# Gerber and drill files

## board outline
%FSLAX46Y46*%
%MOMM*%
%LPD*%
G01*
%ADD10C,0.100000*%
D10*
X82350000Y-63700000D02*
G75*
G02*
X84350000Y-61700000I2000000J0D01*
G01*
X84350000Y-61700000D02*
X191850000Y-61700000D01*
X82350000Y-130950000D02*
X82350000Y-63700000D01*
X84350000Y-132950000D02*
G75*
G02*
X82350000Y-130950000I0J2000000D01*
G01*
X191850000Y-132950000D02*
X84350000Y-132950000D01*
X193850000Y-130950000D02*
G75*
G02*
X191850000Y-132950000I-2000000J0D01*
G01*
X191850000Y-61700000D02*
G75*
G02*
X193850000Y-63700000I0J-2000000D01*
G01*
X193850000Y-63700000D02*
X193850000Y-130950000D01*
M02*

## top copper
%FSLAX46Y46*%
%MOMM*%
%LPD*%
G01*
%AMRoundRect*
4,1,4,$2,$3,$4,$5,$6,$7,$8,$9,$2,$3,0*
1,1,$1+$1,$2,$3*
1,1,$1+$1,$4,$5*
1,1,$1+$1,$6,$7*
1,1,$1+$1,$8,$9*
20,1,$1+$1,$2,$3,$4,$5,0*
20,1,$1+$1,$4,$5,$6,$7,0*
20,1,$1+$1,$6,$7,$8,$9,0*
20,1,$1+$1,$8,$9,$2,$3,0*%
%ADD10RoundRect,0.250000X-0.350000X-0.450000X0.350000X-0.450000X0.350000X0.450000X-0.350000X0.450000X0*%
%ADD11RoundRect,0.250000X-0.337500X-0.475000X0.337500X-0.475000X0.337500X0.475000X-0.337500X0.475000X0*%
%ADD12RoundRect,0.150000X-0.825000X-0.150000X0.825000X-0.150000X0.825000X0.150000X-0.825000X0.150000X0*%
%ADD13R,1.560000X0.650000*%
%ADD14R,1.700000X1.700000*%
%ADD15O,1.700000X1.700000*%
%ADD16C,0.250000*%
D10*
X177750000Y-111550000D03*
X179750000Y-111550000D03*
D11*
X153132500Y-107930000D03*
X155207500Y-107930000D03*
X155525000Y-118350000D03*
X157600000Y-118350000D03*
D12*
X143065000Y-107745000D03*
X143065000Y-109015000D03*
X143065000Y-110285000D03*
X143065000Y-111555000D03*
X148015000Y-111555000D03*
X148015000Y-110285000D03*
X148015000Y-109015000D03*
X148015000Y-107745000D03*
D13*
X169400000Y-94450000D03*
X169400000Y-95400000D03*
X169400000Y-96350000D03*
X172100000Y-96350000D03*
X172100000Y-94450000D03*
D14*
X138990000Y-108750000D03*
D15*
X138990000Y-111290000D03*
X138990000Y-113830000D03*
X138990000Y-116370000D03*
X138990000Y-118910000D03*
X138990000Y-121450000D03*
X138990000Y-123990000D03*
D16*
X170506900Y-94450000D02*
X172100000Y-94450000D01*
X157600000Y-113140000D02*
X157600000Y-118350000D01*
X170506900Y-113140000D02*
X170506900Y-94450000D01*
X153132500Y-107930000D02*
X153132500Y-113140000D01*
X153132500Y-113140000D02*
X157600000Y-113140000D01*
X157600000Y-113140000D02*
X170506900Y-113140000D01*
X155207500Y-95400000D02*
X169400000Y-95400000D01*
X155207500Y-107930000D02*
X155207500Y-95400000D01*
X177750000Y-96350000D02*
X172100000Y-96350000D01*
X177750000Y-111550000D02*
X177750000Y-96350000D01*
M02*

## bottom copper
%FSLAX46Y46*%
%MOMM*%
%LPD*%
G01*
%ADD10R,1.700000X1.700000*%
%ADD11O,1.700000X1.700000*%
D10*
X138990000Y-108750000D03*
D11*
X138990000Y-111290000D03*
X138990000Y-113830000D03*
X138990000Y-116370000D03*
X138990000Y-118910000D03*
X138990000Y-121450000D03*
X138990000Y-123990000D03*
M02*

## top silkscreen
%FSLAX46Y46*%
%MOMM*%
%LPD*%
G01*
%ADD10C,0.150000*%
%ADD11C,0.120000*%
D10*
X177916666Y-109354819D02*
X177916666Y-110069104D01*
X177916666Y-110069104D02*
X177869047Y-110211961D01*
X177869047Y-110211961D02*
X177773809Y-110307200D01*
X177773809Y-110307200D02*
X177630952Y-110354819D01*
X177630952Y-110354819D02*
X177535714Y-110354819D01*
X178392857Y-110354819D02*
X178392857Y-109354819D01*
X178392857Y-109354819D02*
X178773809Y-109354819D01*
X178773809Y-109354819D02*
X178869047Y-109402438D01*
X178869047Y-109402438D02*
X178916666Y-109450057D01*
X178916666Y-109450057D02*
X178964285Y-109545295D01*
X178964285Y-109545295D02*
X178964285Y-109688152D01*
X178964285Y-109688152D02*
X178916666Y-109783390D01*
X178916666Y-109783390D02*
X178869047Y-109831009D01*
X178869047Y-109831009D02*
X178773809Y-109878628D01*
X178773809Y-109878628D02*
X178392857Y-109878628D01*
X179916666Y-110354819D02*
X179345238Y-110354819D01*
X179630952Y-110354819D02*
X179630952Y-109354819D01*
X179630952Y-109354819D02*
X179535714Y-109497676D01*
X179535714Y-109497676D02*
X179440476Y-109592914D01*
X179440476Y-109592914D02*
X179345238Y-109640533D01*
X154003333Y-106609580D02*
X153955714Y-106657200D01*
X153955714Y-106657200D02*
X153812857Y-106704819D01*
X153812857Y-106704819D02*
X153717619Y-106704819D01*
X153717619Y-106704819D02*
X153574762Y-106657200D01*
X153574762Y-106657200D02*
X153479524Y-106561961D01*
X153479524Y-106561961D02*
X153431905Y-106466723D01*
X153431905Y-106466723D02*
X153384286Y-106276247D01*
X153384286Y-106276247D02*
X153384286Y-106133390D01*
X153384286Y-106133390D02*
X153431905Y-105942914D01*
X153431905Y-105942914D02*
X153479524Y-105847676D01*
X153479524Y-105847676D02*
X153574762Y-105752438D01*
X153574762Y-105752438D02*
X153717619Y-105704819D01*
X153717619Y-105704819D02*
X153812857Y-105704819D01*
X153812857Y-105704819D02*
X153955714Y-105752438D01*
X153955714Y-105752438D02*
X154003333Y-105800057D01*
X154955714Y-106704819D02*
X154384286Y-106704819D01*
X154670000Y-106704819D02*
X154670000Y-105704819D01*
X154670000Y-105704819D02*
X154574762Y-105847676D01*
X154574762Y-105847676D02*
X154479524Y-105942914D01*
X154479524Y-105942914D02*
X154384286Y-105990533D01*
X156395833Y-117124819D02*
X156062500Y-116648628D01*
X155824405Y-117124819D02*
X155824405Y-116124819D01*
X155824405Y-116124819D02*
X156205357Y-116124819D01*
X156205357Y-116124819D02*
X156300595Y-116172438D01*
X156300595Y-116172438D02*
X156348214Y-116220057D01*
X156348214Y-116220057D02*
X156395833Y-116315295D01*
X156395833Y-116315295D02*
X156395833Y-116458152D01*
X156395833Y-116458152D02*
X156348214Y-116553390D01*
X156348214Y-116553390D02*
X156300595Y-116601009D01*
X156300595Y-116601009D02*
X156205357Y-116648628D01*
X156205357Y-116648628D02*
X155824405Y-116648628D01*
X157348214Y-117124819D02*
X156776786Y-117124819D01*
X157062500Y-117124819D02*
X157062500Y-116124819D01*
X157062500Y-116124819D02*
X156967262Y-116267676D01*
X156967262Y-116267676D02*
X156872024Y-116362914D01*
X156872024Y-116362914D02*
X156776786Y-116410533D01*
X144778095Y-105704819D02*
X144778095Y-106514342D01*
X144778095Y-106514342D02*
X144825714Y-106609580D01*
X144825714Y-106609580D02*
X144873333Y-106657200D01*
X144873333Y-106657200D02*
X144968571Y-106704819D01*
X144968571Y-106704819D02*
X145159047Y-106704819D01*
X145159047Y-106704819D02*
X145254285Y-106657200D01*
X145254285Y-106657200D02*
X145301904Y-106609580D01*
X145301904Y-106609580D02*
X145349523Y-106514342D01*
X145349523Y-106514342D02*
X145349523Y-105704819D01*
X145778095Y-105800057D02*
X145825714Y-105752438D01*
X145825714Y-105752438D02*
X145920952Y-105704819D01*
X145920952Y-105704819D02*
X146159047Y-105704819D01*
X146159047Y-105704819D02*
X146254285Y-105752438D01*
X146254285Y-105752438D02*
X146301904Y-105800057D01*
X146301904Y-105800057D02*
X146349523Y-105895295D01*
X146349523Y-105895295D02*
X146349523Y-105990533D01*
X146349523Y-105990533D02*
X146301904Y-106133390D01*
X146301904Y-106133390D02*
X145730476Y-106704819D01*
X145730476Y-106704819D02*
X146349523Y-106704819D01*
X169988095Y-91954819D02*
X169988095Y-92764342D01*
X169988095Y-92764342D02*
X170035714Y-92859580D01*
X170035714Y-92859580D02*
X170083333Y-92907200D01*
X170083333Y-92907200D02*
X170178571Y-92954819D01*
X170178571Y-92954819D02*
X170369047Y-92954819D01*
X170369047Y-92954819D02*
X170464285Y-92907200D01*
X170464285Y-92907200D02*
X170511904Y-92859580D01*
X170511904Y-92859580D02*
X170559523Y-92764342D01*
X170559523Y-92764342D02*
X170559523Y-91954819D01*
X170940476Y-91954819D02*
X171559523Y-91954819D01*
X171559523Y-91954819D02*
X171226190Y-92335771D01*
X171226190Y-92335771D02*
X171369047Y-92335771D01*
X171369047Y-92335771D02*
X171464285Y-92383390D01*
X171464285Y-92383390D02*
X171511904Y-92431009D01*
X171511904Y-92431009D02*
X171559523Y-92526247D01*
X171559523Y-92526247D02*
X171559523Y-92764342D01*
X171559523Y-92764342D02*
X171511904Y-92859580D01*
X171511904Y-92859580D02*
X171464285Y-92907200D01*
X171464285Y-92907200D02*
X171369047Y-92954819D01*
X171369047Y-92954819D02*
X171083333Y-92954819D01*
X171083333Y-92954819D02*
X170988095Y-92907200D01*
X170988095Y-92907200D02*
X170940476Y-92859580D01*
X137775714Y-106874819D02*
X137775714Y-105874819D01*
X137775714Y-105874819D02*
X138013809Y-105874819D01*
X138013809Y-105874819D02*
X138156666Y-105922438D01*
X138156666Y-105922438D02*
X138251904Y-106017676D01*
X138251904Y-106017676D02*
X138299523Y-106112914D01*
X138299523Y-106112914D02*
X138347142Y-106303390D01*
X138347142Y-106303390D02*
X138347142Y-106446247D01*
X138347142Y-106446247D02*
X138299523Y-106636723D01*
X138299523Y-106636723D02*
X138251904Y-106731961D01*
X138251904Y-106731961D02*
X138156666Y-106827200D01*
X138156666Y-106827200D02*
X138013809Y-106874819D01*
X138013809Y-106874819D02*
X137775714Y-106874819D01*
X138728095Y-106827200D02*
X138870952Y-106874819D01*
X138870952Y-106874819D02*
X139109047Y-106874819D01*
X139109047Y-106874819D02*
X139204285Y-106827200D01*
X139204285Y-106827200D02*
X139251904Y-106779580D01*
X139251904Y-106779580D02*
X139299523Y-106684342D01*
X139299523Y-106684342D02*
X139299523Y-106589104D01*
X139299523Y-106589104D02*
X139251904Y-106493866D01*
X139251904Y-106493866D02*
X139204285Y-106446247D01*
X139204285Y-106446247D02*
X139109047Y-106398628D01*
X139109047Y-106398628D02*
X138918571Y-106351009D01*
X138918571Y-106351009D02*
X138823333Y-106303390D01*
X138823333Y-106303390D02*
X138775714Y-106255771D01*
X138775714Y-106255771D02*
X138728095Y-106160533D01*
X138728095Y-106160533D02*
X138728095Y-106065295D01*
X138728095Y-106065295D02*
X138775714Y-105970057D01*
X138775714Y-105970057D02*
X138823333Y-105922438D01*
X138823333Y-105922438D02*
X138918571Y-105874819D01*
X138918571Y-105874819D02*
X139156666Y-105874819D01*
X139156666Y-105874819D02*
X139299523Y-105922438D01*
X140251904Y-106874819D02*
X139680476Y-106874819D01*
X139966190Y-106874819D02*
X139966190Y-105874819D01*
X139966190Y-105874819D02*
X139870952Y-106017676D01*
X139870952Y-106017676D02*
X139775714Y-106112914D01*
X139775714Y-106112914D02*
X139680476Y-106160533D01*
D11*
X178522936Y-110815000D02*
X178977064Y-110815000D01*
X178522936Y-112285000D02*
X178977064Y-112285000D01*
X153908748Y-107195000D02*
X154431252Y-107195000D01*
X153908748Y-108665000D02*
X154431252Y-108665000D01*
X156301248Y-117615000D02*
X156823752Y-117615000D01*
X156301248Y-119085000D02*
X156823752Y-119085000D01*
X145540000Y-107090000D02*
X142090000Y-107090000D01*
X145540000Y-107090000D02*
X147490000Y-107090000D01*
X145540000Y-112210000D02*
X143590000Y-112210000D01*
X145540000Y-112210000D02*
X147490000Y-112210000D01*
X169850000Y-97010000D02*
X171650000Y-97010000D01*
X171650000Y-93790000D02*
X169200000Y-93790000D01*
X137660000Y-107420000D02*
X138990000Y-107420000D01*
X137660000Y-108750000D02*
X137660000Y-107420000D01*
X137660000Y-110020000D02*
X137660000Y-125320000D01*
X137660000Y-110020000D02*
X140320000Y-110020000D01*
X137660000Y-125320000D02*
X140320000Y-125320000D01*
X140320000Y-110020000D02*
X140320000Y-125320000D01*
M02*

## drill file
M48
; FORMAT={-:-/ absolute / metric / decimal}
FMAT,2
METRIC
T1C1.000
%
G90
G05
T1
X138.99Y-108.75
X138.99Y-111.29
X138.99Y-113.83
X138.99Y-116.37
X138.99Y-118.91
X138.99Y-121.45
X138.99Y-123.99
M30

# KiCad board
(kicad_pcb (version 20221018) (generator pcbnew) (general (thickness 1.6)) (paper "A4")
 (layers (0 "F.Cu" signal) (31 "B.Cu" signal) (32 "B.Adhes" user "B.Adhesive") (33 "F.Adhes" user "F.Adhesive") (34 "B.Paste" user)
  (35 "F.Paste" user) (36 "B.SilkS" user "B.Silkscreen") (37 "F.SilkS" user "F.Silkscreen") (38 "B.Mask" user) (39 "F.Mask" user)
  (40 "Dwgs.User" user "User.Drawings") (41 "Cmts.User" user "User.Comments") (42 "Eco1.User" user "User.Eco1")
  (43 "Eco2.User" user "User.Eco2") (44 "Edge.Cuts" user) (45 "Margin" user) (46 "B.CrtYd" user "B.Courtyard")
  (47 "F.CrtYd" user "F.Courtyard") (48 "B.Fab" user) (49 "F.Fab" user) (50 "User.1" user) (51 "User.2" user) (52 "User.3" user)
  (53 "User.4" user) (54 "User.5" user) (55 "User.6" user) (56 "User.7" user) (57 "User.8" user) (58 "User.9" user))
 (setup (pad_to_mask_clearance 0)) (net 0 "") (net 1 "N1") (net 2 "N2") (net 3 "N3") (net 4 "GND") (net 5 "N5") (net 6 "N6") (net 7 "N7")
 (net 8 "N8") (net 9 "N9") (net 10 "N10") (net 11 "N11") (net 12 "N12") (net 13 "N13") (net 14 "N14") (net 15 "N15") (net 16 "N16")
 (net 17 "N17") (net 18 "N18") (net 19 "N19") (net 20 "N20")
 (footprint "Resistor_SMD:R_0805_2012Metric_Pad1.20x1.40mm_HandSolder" (layer "F.Cu") (at 178.75 111.55)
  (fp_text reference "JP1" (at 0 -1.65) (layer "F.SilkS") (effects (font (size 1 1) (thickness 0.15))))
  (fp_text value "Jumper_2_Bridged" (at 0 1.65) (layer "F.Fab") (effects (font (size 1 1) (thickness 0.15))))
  (fp_line (start -0.227064 -0.735) (end 0.227064 -0.735) (stroke (width 0.12) (type solid)) (layer "F.SilkS"))
  (fp_line (start -0.227064 0.735) (end 0.227064 0.735) (stroke (width 0.12) (type solid)) (layer "F.SilkS"))
  (pad "1" smd roundrect (at -1 0) (size 1.2 1.4) (layers "F.Cu" "F.Paste" "F.Mask") (roundrect_rratio 0.208333) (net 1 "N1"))
  (pad "2" smd roundrect (at 1 0) (size 1.2 1.4) (layers "F.Cu" "F.Paste" "F.Mask") (roundrect_rratio 0.208333) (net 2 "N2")))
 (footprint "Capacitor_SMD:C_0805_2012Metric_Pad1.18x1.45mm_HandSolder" (layer "F.Cu") (at 154.17 107.93)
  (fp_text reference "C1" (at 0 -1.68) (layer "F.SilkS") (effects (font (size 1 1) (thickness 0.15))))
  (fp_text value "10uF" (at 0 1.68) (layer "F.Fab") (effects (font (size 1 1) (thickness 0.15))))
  (fp_line (start -0.261252 -0.735) (end 0.261252 -0.735) (stroke (width 0.12) (type solid)) (layer "F.SilkS"))
  (fp_line (start -0.261252 0.735) (end 0.261252 0.735) (stroke (width 0.12) (type solid)) (layer "F.SilkS"))
  (pad "1" smd roundrect (at -1.0375 0) (size 1.175 1.45) (layers "F.Cu" "F.Paste" "F.Mask") (roundrect_rratio 0.212766) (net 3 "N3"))
  (pad "2" smd roundrect (at 1.0375 0) (size 1.175 1.45) (layers "F.Cu" "F.Paste" "F.Mask") (roundrect_rratio 0.212766) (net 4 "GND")))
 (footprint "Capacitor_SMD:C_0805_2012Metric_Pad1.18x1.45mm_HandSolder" (layer "F.Cu") (at 156.5625 118.35)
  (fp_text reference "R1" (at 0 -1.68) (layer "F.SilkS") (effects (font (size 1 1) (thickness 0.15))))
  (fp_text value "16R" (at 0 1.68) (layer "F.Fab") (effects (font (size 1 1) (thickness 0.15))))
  (fp_line (start -0.261252 -0.735) (end 0.261252 -0.735) (stroke (width 0.12) (type solid)) (layer "F.SilkS"))
  (fp_line (start -0.261252 0.735) (end 0.261252 0.735) (stroke (width 0.12) (type solid)) (layer "F.SilkS"))
  (pad "1" smd roundrect (at -1.0375 0) (size 1.175 1.45) (layers "F.Cu" "F.Paste" "F.Mask") (roundrect_rratio 0.212766) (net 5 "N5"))
  (pad "2" smd roundrect (at 1.0375 0) (size 1.175 1.45) (layers "F.Cu" "F.Paste" "F.Mask") (roundrect_rratio 0.212766) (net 3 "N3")))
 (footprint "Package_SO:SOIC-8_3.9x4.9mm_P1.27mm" (layer "F.Cu") (at 145.54 109.65)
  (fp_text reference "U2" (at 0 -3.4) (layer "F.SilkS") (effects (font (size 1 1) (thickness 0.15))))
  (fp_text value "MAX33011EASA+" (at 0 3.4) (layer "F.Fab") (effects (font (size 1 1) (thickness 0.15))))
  (fp_line (start 0 -2.56) (end -3.45 -2.56) (stroke (width 0.12) (type solid)) (layer "F.SilkS"))
  (fp_line (start 0 -2.56) (end 1.95 -2.56) (stroke (width 0.12) (type solid)) (layer "F.SilkS"))
  (fp_line (start 0 2.56) (end -1.95 2.56) (stroke (width 0.12) (type solid)) (layer "F.SilkS"))
  (fp_line (start 0 2.56) (end 1.95 2.56) (stroke (width 0.12) (type solid)) (layer "F.SilkS"))
  (pad "1" smd roundrect (at -2.475 -1.905) (size 1.95 0.6) (layers "F.Cu" "F.Paste" "F.Mask") (roundrect_rratio 0.25) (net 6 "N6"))
  (pad "2" smd roundrect (at -2.475 -0.635) (size 1.95 0.6) (layers "F.Cu" "F.Paste" "F.Mask") (roundrect_rratio 0.25) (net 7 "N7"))
  (pad "3" smd roundrect (at -2.475 0.635) (size 1.95 0.6) (layers "F.Cu" "F.Paste" "F.Mask") (roundrect_rratio 0.25) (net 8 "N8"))
  (pad "4" smd roundrect (at -2.475 1.905) (size 1.95 0.6) (layers "F.Cu" "F.Paste" "F.Mask") (roundrect_rratio 0.25) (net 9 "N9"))
  (pad "5" smd roundrect (at 2.475 1.905) (size 1.95 0.6) (layers "F.Cu" "F.Paste" "F.Mask") (roundrect_rratio 0.25) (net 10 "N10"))
  (pad "6" smd roundrect (at 2.475 0.635) (size 1.95 0.6) (layers "F.Cu" "F.Paste" "F.Mask") (roundrect_rratio 0.25) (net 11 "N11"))
  (pad "7" smd roundrect (at 2.475 -0.635) (size 1.95 0.6) (layers "F.Cu" "F.Paste" "F.Mask") (roundrect_rratio 0.25) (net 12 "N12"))
  (pad "8" smd roundrect (at 2.475 -1.905) (size 1.95 0.6) (layers "F.Cu" "F.Paste" "F.Mask") (roundrect_rratio 0.25) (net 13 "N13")))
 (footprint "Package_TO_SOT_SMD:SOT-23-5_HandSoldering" (layer "F.Cu") (at 170.75 95.4)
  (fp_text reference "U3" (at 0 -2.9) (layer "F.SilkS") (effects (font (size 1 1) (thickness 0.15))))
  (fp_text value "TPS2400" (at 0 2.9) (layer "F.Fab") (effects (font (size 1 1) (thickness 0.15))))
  (fp_line (start -0.9 1.61) (end 0.9 1.61) (stroke (width 0.12) (type solid)) (layer "F.SilkS"))
  (fp_line (start 0.9 -1.61) (end -1.55 -1.61) (stroke (width 0.12) (type solid)) (layer "F.SilkS"))
  (pad "1" smd rect (at -1.35 -0.95) (size 1.56 0.65) (layers "F.Cu" "F.Paste" "F.Mask"))
  (pad "2" smd rect (at -1.35 0) (size 1.56 0.65) (layers "F.Cu" "F.Paste" "F.Mask") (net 4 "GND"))
  (pad "3" smd rect (at -1.35 0.95) (size 1.56 0.65) (layers "F.Cu" "F.Paste" "F.Mask"))
  (pad "4" smd rect (at 1.35 0.95) (size 1.56 0.65) (layers "F.Cu" "F.Paste" "F.Mask") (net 1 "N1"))
  (pad "5" smd rect (at 1.35 -0.95) (size 1.56 0.65) (layers "F.Cu" "F.Paste" "F.Mask") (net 3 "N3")))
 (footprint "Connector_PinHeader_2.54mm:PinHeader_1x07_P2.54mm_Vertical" (layer "F.Cu") (at 138.99 108.75)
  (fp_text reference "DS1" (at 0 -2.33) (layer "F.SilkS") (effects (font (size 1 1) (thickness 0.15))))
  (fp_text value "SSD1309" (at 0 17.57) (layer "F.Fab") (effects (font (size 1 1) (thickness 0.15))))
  (fp_line (start -1.33 -1.33) (end 0 -1.33) (stroke (width 0.12) (type solid)) (layer "F.SilkS"))
  (fp_line (start -1.33 0) (end -1.33 -1.33) (stroke (width 0.12) (type solid)) (layer "F.SilkS"))
  (fp_line (start -1.33 1.27) (end -1.33 16.57) (stroke (width 0.12) (type solid)) (layer "F.SilkS"))
  (fp_line (start -1.33 1.27) (end 1.33 1.27) (stroke (width 0.12) (type solid)) (layer "F.SilkS"))
  (fp_line (start -1.33 16.57) (end 1.33 16.57) (stroke (width 0.12) (type solid)) (layer "F.SilkS"))
  (fp_line (start 1.33 1.27) (end 1.33 16.57) (stroke (width 0.12) (type solid)) (layer "F.SilkS"))
  (pad "1" thru_hole rect (at 0 0) (size 1.7 1.7) (drill 1) (layers "*.Cu" "*.Mask") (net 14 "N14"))
  (pad "2" thru_hole oval (at 0 2.54) (size 1.7 1.7) (drill 1) (layers "*.Cu" "*.Mask") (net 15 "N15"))
  (pad "3" thru_hole oval (at 0 5.08) (size 1.7 1.7) (drill 1) (layers "*.Cu" "*.Mask") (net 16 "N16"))
  (pad "4" thru_hole oval (at 0 7.62) (size 1.7 1.7) (drill 1) (layers "*.Cu" "*.Mask") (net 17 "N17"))
  (pad "5" thru_hole oval (at 0 10.16) (size 1.7 1.7) (drill 1) (layers "*.Cu" "*.Mask") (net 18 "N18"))
  (pad "6" thru_hole oval (at 0 12.7) (size 1.7 1.7) (drill 1) (layers "*.Cu" "*.Mask") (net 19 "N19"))
  (pad "7" thru_hole oval (at 0 15.24) (size 1.7 1.7) (drill 1) (layers "*.Cu" "*.Mask") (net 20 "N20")))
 (gr_arc (start 82.35 63.7) (mid 82.935786 62.285786) (end 84.35 61.7) (stroke (width 0.1) (type default)) (layer "Edge.Cuts"))
 (gr_line (start 84.35 61.7) (end 191.85 61.7) (stroke (width 0.1) (type default)) (layer "Edge.Cuts"))
 (gr_line (start 82.35 130.95) (end 82.35 63.7) (stroke (width 0.1) (type default)) (layer "Edge.Cuts"))
 (gr_arc (start 84.35 132.95) (mid 82.935786 132.364214) (end 82.35 130.95) (stroke (width 0.1) (type default)) (layer "Edge.Cuts"))
 (gr_line (start 191.85 132.95) (end 84.35 132.95) (stroke (width 0.1) (type default)) (layer "Edge.Cuts"))
 (gr_arc (start 193.85 130.95) (mid 193.264214 132.364214) (end 191.85 132.95) (stroke (width 0.1) (type default)) (layer "Edge.Cuts"))
 (gr_arc (start 191.85 61.7) (mid 193.264214 62.285786) (end 193.85 63.7) (stroke (width 0.1) (type default)) (layer "Edge.Cuts"))
 (gr_line (start 193.85 63.7) (end 193.85 130.95) (stroke (width 0.1) (type default)) (layer "Edge.Cuts"))
 (segment (start 170.5069 94.45) (end 172.1 94.45) (width 0.25) (layer "F.Cu") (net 3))
 (segment (start 157.6 113.14) (end 157.6 118.35) (width 0.25) (layer "F.Cu") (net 3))
 (segment (start 170.5069 113.14) (end 170.5069 94.45) (width 0.25) (layer "F.Cu") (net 3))
 (segment (start 153.1325 107.93) (end 153.1325 113.14) (width 0.25) (layer "F.Cu") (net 3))
 (segment (start 153.1325 113.14) (end 157.6 113.14) (width 0.25) (layer "F.Cu") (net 3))
 (segment (start 157.6 113.14) (end 170.5069 113.14) (width 0.25) (layer "F.Cu") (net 3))
 (segment (start 155.2075 95.4) (end 169.4 95.4) (width 0.25) (layer "F.Cu") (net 4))
 (segment (start 155.2075 107.93) (end 155.2075 95.4) (width 0.25) (layer "F.Cu") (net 4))
 (segment (start 177.75 96.35) (end 172.1 96.35) (width 0.25) (layer "F.Cu") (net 1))
 (segment (start 177.75 111.55) (end 177.75 96.35) (width 0.25) (layer "F.Cu") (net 1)))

